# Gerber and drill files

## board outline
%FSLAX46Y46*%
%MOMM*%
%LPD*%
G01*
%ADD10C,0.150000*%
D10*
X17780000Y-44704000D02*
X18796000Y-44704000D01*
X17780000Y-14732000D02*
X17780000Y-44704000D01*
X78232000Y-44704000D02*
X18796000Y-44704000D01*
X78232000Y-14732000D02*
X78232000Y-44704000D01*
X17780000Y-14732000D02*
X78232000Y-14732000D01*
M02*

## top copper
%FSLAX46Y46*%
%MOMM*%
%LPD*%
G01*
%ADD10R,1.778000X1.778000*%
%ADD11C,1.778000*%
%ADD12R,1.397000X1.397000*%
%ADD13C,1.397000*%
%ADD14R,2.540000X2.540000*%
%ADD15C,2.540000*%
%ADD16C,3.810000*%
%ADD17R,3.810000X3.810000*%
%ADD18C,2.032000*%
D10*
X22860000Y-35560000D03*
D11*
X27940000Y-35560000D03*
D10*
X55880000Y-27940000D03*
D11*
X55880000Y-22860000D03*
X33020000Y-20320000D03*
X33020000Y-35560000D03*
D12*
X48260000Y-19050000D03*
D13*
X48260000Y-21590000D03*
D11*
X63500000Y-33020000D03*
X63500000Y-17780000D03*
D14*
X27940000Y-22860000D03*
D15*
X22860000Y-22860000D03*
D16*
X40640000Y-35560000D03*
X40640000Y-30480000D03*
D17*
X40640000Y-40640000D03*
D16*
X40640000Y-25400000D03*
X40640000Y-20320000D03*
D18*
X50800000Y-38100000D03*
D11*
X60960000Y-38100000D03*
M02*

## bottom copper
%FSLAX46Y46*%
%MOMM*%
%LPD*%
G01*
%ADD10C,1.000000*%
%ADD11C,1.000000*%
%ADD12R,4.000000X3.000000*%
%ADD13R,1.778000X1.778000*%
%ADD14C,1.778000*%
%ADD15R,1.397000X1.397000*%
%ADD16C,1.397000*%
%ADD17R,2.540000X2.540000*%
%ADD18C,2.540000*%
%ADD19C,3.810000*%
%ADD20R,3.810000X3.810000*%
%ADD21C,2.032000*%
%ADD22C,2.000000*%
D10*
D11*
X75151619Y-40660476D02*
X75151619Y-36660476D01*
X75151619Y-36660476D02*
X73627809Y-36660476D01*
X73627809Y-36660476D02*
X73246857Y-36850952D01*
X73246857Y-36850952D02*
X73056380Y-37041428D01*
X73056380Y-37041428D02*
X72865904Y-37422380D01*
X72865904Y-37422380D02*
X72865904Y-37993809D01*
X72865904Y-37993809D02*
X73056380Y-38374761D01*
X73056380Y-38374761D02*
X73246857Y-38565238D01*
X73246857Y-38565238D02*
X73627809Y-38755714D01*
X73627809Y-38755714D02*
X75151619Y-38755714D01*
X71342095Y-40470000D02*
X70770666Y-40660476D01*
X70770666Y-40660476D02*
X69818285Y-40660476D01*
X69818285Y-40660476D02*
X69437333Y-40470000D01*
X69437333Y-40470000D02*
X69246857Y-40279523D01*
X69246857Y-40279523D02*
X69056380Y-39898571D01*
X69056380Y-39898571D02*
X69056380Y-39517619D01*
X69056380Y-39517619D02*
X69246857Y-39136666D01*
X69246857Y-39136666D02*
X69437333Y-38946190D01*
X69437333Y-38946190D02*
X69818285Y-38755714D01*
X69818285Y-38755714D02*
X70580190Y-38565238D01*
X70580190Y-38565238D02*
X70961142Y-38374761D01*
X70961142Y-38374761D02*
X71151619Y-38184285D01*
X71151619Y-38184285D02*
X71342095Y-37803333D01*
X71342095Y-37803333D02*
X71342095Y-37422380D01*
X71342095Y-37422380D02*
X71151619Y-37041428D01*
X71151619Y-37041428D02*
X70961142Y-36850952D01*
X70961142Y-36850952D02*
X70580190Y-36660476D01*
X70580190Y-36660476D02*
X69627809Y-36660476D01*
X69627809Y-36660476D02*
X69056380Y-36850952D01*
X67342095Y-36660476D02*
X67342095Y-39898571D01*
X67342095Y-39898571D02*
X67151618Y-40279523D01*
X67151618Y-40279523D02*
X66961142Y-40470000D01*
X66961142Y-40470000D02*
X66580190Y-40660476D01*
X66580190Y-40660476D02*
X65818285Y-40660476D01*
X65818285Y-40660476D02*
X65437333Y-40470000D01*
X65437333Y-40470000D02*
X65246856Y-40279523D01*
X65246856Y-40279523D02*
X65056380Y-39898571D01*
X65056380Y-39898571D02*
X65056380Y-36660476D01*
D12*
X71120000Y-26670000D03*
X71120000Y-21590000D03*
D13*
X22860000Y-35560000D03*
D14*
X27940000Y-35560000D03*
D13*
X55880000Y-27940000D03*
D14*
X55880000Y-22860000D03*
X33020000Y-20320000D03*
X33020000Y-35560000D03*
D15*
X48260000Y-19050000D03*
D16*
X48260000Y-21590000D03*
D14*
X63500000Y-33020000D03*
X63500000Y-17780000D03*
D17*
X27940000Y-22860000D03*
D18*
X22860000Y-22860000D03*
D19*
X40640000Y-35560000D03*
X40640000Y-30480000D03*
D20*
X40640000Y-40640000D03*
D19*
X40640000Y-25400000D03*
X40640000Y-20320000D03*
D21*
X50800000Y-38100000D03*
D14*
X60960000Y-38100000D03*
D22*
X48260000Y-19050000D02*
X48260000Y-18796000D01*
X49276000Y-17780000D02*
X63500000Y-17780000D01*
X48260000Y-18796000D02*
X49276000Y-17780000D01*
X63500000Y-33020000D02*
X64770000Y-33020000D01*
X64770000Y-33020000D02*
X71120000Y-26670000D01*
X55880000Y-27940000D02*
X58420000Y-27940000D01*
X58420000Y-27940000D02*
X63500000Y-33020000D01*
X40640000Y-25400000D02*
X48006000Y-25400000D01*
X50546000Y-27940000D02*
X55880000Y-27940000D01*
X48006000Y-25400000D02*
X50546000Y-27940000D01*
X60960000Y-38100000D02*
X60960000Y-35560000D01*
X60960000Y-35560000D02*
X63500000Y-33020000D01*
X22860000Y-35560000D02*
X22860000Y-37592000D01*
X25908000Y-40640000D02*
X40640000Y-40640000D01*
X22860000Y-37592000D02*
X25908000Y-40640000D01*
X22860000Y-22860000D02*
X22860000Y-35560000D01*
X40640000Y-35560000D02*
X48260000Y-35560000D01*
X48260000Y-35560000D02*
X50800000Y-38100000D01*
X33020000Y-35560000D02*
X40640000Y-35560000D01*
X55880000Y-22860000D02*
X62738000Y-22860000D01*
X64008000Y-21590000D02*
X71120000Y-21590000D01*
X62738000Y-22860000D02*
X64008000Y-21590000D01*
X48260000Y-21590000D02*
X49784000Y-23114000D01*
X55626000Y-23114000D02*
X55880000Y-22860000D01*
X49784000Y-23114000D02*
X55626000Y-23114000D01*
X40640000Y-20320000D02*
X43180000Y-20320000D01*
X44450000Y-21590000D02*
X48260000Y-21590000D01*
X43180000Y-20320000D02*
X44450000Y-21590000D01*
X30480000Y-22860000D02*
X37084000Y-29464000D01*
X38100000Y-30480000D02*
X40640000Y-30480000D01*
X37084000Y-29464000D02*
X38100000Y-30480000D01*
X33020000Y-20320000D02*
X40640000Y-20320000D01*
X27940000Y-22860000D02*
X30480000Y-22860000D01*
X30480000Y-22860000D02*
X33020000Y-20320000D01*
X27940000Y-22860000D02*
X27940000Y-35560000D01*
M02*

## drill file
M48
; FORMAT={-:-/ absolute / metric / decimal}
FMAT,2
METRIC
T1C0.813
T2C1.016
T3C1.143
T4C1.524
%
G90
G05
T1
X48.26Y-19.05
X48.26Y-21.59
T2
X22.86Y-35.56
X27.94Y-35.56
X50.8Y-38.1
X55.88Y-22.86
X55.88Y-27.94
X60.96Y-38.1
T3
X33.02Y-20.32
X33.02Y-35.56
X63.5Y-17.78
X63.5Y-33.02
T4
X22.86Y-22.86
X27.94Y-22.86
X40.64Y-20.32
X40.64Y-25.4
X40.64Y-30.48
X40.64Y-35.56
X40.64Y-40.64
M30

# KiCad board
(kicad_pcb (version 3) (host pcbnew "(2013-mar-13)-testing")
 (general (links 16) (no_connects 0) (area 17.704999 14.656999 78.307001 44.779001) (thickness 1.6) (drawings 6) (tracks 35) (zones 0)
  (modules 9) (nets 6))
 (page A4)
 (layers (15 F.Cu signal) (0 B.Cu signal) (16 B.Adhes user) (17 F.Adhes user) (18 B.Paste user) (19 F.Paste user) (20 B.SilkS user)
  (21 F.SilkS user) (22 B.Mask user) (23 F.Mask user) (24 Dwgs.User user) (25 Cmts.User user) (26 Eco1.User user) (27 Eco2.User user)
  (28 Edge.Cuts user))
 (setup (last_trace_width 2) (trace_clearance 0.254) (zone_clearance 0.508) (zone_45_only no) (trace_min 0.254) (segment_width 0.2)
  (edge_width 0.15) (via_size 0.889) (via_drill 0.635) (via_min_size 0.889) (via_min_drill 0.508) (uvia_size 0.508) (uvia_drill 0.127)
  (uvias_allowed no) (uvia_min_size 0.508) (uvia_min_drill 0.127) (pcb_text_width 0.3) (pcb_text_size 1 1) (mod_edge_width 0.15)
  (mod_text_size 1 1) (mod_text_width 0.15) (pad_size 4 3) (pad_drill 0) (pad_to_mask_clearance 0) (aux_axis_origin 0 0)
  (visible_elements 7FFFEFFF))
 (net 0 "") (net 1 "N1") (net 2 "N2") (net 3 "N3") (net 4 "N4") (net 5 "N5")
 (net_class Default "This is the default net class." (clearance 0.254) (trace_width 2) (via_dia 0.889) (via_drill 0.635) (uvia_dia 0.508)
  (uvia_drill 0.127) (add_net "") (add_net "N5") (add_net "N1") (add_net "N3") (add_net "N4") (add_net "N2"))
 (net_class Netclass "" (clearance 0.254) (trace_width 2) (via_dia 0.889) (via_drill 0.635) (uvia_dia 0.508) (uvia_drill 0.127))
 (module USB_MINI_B (layer F.Cu) (at 71.12 24.13 180)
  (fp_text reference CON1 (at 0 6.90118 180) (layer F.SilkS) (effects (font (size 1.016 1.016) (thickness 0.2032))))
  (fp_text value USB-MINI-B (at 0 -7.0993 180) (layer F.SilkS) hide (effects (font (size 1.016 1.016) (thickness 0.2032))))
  (pad 1 smd rect (at 0 -2.54 180) (size 4 3) (layers *.Adhes *.Paste *.SilkS *.Mask B.Cu Dwgs.User Eco1.User Eco2.User) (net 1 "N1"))
  (pad 5 smd rect (at 0 2.54 180) (size 4 3) (layers *.Adhes *.Paste *.SilkS *.Mask B.Cu Dwgs.User Eco1.User Eco2.User) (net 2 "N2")))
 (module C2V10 (layer F.Cu) (at 25.4 35.56)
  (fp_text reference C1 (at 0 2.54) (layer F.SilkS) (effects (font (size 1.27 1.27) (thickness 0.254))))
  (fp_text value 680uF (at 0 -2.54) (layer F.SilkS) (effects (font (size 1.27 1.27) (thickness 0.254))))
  (pad 1 thru_hole rect (at -2.54 0) (size 1.778 1.778) (drill 1.016) (layers *.Cu *.Mask F.SilkS) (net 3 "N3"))
  (pad 2 thru_hole circle (at 2.54 0) (size 1.778 1.778) (drill 1.016) (layers *.Cu *.Mask F.SilkS) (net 2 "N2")))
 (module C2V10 (layer F.Cu) (at 55.88 25.4 90)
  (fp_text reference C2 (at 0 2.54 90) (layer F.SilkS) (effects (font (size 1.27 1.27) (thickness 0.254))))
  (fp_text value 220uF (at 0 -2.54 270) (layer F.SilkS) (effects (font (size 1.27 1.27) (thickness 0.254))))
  (pad 1 thru_hole rect (at -2.54 0 90) (size 1.778 1.778) (drill 1.016) (layers *.Cu *.Mask F.SilkS) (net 1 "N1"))
  (pad 2 thru_hole circle (at 2.54 0 90) (size 1.778 1.778) (drill 1.016) (layers *.Cu *.Mask F.SilkS) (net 2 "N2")))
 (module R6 (layer F.Cu) (at 33.02 27.94 270) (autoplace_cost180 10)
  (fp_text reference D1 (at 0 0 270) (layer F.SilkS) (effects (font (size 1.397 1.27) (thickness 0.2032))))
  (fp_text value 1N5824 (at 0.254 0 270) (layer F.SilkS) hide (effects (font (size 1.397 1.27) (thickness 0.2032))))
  (pad 1 thru_hole circle (at -7.62 0 270) (size 1.778 1.778) (drill 1.143) (layers *.Cu *.Mask F.SilkS) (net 2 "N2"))
  (pad 2 thru_hole circle (at 7.62 0 270) (size 1.778 1.778) (drill 1.143) (layers *.Cu *.Mask F.SilkS) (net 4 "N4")))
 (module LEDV (layer F.Cu) (at 48.26 20.32 270)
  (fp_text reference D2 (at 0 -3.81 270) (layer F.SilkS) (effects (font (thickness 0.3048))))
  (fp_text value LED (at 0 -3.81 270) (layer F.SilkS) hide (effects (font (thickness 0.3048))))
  (pad 1 thru_hole rect (at -1.27 0 270) (size 1.397 1.397) (drill 0.8128) (layers *.Cu *.Mask F.SilkS) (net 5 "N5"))
  (pad 2 thru_hole circle (at 1.27 0 270) (size 1.397 1.397) (drill 0.8128) (layers *.Cu *.Mask F.SilkS) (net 2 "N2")))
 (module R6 (layer F.Cu) (at 63.5 25.4 90) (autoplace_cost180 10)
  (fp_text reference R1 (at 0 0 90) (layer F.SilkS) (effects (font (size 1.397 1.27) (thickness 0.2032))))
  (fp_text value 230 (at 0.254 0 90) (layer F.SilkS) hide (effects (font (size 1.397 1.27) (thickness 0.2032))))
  (pad 1 thru_hole circle (at -7.62 0 90) (size 1.778 1.778) (drill 1.143) (layers *.Cu *.Mask F.SilkS) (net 1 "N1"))
  (pad 2 thru_hole circle (at 7.62 0 90) (size 1.778 1.778) (drill 1.143) (layers *.Cu *.Mask F.SilkS) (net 5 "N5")))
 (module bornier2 (layer F.Cu) (at 25.4 22.86 180)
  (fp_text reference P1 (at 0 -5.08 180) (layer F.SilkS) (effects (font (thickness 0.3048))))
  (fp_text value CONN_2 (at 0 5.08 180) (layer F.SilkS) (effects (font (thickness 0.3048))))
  (pad 1 thru_hole rect (at -2.54 0 180) (size 2.54 2.54) (drill 1.524) (layers *.Cu *.Mask F.SilkS) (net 2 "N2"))
  (pad 2 thru_hole circle (at 2.54 0 180) (size 2.54 2.54) (drill 1.524) (layers *.Cu *.Mask F.SilkS) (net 3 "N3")))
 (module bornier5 (layer F.Cu) (at 40.64 30.48 90)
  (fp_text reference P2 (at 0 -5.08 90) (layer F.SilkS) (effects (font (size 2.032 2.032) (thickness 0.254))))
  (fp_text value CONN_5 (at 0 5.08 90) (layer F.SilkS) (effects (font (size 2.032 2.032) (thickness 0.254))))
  (pad 2 thru_hole circle (at -5.08 0 90) (size 3.81 3.81) (drill 1.524) (layers *.Cu *.Mask F.SilkS) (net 4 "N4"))
  (pad 3 thru_hole circle (at 0 0 90) (size 3.81 3.81) (drill 1.524) (layers *.Cu *.Mask F.SilkS) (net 2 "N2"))
  (pad 1 thru_hole rect (at -10.16 0 90) (size 3.81 3.81) (drill 1.524) (layers *.Cu *.Mask F.SilkS) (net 3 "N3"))
  (pad 4 thru_hole circle (at 5.08 0 90) (size 3.81 3.81) (drill 1.524) (layers *.Cu *.Mask F.SilkS) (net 1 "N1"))
  (pad 5 thru_hole circle (at 10.16 0 90) (size 3.81 3.81) (drill 1.524) (layers *.Cu *.Mask F.SilkS) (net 2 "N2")))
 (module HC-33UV (layer F.Cu) (at 55.88 38.1) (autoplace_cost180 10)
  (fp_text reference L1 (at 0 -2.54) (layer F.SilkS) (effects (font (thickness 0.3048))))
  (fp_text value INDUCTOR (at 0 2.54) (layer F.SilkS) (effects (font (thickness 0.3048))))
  (pad 1 thru_hole circle (at -5.08 0) (size 2.032 2.032) (drill 1.016) (layers *.Cu *.Mask F.SilkS) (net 4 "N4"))
  (pad 2 thru_hole circle (at 5.08 0) (size 1.778 1.778) (drill 1.016) (layers *.Cu *.Mask F.SilkS) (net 1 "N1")))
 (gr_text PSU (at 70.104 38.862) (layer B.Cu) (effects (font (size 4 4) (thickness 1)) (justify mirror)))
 (gr_line (start 17.78 44.704) (end 18.796 44.704) (angle 90) (layer Edge.Cuts) (width 0.15))
 (gr_line (start 17.78 14.732) (end 17.78 44.704) (angle 90) (layer Edge.Cuts) (width 0.15))
 (gr_line (start 78.232 44.704) (end 18.796 44.704) (angle 90) (layer Edge.Cuts) (width 0.15))
 (gr_line (start 78.232 14.732) (end 78.232 44.704) (angle 90) (layer Edge.Cuts) (width 0.15))
 (gr_line (start 17.78 14.732) (end 78.232 14.732) (angle 90) (layer Edge.Cuts) (width 0.15))
 (segment (start 48.26 19.05) (end 48.26 18.796) (width 2) (layer B.Cu) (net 5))
 (segment (start 49.276 17.78) (end 63.5 17.78) (width 2) (layer B.Cu) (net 5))
 (segment (start 48.26 18.796) (end 49.276 17.78) (width 2) (layer B.Cu) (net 5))
 (segment (start 63.5 33.02) (end 64.77 33.02) (width 2) (layer B.Cu) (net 1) (status 400000))
 (segment (start 64.77 33.02) (end 71.12 26.67) (width 2) (layer B.Cu) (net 1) (status 800000))
 (segment (start 55.88 27.94) (end 58.42 27.94) (width 2) (layer B.Cu) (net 1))
 (segment (start 58.42 27.94) (end 63.5 33.02) (width 2) (layer B.Cu) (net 1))
 (segment (start 40.64 25.4) (end 48.006 25.4) (width 2) (layer B.Cu) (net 1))
 (segment (start 50.546 27.94) (end 55.88 27.94) (width 2) (layer B.Cu) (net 1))
 (segment (start 48.006 25.4) (end 50.546 27.94) (width 2) (layer B.Cu) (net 1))
 (segment (start 60.96 38.1) (end 60.96 35.56) (width 2) (layer B.Cu) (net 1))
 (segment (start 60.96 35.56) (end 63.5 33.02) (width 2) (layer B.Cu) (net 1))
 (segment (start 22.86 35.56) (end 22.86 37.592) (width 2) (layer B.Cu) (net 3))
 (segment (start 25.908 40.64) (end 40.64 40.64) (width 2) (layer B.Cu) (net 3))
 (segment (start 22.86 37.592) (end 25.908 40.64) (width 2) (layer B.Cu) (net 3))
 (segment (start 22.86 22.86) (end 22.86 35.56) (width 2) (layer B.Cu) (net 3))
 (segment (start 40.64 35.56) (end 48.26 35.56) (width 2) (layer B.Cu) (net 4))
 (segment (start 48.26 35.56) (end 50.8 38.1) (width 2) (layer B.Cu) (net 4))
 (segment (start 33.02 35.56) (end 40.64 35.56) (width 2) (layer B.Cu) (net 4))
 (segment (start 55.88 22.86) (end 62.738 22.86) (width 2) (layer B.Cu) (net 2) (status 400000))
 (segment (start 64.008 21.59) (end 71.12 21.59) (width 2) (layer B.Cu) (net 2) (status 800000))
 (segment (start 62.738 22.86) (end 64.008 21.59) (width 2) (layer B.Cu) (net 2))
 (segment (start 48.26 21.59) (end 49.784 23.114) (width 2) (layer B.Cu) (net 2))
 (segment (start 55.626 23.114) (end 55.88 22.86) (width 2) (layer B.Cu) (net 2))
 (segment (start 49.784 23.114) (end 55.626 23.114) (width 2) (layer B.Cu) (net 2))
 (segment (start 40.64 20.32) (end 43.18 20.32) (width 2) (layer B.Cu) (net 2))
 (segment (start 44.45 21.59) (end 48.26 21.59) (width 2) (layer B.Cu) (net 2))
 (segment (start 43.18 20.32) (end 44.45 21.59) (width 2) (layer B.Cu) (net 2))
 (segment (start 30.48 22.86) (end 37.084 29.464) (width 2) (layer B.Cu) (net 2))
 (segment (start 38.1 30.48) (end 40.64 30.48) (width 2) (layer B.Cu) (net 2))
 (segment (start 37.084 29.464) (end 38.1 30.48) (width 2) (layer B.Cu) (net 2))
 (segment (start 33.02 20.32) (end 40.64 20.32) (width 2) (layer B.Cu) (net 2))
 (segment (start 27.94 22.86) (end 30.48 22.86) (width 2) (layer B.Cu) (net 2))
 (segment (start 30.48 22.86) (end 33.02 20.32) (width 2) (layer B.Cu) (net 2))
 (segment (start 27.94 22.86) (end 27.94 35.56) (width 2) (layer B.Cu) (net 2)))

